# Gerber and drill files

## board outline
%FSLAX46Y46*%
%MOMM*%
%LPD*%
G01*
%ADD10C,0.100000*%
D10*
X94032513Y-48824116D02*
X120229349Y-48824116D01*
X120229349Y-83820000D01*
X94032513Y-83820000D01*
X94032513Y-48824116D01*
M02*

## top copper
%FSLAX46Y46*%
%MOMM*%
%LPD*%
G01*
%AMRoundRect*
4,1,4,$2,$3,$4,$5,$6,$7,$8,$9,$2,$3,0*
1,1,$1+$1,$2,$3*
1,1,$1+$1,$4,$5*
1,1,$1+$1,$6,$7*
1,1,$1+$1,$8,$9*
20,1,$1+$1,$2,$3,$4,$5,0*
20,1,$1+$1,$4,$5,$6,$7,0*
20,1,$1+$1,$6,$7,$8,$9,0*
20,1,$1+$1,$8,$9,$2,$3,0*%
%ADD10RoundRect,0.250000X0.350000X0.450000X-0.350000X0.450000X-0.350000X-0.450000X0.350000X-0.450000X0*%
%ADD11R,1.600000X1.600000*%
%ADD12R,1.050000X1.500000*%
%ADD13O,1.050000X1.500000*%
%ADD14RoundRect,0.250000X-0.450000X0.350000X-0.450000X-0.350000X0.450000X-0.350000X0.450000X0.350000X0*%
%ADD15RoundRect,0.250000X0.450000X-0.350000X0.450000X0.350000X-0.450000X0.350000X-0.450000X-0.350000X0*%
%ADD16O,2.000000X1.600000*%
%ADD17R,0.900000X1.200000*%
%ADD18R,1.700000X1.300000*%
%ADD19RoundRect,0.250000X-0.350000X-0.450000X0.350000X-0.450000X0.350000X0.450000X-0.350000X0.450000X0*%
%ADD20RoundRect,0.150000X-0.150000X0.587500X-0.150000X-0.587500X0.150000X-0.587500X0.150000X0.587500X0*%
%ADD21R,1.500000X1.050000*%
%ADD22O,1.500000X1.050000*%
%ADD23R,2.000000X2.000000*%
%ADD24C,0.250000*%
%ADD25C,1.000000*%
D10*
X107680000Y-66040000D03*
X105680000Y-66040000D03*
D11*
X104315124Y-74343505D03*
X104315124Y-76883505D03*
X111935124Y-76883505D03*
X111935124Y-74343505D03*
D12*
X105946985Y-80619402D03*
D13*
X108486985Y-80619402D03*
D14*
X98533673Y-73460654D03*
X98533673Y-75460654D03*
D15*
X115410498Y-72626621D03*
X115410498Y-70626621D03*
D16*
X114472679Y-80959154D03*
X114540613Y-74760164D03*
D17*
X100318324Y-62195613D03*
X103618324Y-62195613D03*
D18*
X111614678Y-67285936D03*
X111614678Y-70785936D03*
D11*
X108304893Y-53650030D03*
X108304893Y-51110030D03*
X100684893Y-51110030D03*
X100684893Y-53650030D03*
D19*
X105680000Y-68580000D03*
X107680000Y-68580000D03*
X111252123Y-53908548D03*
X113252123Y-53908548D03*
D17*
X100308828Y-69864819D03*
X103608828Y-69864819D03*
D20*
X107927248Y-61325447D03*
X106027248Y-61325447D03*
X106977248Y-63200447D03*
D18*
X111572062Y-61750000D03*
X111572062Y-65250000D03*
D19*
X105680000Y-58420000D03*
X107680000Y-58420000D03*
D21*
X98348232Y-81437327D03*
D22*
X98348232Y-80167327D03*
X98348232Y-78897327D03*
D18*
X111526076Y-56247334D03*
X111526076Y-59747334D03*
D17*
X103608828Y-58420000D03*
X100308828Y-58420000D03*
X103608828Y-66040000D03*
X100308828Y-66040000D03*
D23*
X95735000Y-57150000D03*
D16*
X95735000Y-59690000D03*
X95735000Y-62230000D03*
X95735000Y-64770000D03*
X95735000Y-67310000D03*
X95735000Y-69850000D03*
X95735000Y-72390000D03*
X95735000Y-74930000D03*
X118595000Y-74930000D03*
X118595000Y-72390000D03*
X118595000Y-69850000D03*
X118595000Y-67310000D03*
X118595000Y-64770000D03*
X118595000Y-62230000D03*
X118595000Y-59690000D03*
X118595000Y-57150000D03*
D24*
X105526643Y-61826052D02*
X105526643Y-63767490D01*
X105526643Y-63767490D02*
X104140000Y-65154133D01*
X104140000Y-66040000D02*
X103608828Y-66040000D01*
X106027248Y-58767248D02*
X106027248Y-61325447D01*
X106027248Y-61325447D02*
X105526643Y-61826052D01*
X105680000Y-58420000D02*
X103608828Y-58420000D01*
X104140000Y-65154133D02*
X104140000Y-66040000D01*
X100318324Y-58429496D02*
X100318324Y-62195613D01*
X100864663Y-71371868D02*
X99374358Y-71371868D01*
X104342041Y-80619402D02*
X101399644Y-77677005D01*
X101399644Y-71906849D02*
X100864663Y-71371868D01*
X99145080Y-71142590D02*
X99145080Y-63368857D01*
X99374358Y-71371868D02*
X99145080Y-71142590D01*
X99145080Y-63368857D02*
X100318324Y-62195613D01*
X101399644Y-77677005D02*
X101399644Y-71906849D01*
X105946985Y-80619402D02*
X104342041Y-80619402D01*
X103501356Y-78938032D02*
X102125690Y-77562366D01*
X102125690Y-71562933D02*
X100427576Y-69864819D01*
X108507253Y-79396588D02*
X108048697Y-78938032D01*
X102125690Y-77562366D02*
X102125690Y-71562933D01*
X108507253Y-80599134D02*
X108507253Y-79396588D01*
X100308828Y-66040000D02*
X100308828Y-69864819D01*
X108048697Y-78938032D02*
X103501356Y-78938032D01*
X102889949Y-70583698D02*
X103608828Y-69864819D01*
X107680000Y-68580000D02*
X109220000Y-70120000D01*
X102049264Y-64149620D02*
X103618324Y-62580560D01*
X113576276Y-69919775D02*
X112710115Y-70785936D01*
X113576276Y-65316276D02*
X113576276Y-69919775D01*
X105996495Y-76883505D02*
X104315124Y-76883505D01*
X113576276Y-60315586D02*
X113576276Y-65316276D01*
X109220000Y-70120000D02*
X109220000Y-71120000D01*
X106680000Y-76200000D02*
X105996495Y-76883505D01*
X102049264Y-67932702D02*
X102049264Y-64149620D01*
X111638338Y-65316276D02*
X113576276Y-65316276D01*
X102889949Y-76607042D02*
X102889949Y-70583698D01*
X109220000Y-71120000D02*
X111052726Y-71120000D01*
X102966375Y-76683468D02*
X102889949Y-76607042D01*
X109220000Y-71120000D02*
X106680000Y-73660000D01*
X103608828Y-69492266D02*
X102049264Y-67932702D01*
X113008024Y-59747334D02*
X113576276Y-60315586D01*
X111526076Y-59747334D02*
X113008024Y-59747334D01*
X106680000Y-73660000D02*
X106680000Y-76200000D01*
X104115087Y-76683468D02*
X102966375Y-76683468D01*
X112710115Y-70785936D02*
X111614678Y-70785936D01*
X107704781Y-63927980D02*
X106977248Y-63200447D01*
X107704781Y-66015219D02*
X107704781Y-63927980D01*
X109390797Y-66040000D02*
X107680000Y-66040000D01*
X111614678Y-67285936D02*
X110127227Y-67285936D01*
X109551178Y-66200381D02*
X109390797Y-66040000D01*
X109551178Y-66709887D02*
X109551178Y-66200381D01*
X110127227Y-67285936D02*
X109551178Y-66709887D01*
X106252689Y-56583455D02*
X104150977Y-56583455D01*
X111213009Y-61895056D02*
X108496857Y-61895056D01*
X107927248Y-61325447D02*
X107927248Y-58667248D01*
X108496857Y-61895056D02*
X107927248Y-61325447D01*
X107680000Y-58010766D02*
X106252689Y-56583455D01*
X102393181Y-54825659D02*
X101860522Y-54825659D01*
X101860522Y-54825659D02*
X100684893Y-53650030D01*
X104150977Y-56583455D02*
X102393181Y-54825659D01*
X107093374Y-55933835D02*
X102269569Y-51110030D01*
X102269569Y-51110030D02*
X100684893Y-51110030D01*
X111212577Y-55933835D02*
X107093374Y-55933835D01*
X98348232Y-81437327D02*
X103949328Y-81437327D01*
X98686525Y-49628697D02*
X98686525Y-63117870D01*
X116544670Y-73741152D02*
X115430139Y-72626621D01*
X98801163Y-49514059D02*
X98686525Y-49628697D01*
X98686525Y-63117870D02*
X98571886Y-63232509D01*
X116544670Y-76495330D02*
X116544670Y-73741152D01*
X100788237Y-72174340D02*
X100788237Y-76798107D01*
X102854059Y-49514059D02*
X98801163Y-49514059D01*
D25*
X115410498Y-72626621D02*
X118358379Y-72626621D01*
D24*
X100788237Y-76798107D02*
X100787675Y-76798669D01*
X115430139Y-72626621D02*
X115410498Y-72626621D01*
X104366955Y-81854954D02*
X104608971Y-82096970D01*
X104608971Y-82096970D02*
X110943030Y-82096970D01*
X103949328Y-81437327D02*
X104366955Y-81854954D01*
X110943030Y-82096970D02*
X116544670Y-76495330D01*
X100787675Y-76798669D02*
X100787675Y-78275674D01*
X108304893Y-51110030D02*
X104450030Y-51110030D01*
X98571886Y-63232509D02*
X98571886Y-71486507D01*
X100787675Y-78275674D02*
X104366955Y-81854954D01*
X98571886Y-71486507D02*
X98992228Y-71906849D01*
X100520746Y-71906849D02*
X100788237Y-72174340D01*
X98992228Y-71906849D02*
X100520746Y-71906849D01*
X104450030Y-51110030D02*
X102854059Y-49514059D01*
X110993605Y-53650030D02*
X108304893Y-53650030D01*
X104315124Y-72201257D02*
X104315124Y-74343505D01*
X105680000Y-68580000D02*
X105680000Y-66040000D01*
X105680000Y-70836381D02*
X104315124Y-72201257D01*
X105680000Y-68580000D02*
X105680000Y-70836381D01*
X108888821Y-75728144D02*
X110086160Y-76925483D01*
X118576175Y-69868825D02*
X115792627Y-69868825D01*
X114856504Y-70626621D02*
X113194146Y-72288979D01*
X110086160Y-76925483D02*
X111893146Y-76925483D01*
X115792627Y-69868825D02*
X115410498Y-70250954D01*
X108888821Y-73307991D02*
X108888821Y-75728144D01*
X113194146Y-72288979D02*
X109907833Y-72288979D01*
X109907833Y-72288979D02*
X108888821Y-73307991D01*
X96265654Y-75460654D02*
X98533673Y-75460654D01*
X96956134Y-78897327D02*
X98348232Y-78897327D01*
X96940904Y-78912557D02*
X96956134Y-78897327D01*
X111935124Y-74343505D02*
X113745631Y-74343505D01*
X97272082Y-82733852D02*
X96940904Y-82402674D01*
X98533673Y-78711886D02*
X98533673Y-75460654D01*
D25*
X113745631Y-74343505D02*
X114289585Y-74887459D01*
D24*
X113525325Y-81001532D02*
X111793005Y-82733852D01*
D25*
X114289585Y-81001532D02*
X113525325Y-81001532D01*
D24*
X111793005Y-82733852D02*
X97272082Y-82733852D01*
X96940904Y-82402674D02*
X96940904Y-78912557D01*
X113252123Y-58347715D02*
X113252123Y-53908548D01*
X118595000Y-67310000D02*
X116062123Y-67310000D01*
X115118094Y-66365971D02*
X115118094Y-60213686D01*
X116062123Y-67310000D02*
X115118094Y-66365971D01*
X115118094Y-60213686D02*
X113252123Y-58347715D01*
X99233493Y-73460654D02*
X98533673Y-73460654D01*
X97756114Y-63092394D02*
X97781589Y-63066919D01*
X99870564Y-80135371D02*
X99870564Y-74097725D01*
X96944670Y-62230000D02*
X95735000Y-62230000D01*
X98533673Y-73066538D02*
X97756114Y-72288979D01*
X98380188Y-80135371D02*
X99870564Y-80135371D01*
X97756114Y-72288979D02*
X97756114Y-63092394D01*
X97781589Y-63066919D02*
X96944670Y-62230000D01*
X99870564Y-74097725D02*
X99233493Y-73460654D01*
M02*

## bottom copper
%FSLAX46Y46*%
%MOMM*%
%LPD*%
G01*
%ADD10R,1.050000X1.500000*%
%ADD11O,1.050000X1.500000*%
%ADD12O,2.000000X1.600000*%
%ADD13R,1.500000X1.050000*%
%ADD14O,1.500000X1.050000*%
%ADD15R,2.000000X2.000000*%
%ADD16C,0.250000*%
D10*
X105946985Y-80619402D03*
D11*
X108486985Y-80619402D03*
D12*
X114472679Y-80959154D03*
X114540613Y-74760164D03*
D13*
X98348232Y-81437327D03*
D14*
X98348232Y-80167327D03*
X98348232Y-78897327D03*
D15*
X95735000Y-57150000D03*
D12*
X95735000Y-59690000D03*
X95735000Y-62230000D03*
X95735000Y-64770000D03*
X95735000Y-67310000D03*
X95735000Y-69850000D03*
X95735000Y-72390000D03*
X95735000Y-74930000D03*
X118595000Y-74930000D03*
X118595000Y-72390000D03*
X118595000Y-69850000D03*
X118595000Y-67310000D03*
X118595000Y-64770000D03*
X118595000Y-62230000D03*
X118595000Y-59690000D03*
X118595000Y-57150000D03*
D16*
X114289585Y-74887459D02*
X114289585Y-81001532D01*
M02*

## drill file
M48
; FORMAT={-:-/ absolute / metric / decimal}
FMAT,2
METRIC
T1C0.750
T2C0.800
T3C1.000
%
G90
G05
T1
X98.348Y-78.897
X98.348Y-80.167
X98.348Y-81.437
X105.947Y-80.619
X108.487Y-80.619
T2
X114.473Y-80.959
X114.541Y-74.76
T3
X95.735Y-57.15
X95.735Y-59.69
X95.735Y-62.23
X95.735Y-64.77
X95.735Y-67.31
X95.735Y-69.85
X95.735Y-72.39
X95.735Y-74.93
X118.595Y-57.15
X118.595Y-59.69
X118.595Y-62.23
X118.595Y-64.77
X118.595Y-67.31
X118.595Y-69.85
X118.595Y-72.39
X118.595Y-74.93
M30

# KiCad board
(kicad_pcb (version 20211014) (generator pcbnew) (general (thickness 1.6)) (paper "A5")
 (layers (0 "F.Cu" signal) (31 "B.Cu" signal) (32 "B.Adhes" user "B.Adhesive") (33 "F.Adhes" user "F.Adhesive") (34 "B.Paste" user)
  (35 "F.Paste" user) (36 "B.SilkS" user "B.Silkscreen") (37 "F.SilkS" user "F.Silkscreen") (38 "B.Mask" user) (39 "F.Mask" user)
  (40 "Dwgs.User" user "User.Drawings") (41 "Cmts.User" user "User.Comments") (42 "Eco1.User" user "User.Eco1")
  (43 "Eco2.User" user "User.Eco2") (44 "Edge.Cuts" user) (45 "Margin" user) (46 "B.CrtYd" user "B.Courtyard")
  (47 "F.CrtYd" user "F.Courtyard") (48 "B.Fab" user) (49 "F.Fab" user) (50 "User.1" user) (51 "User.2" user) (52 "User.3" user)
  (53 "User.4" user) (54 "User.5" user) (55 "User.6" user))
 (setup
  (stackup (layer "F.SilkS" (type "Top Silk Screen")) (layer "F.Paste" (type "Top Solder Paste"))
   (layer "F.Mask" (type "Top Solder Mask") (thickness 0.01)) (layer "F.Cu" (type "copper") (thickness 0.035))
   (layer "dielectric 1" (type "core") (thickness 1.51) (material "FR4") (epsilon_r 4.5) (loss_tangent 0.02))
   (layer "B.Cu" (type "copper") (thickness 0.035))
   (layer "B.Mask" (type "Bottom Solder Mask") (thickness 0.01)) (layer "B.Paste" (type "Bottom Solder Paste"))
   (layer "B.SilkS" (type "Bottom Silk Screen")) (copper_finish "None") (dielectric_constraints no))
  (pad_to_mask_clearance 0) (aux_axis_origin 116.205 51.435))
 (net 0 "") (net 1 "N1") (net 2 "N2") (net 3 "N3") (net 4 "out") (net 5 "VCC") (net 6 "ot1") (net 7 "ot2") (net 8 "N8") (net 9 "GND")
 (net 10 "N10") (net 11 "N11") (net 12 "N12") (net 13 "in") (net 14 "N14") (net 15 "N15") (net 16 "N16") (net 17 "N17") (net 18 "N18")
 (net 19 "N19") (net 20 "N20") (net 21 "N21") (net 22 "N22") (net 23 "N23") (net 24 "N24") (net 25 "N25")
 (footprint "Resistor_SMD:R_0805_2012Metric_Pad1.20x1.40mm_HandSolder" (layer "F.Cu") (at 106.68 66.04 180)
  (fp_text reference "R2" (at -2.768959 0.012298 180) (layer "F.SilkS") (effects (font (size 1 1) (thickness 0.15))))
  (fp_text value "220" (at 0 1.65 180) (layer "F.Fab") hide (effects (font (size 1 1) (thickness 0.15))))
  (pad "1" smd roundrect (at -1 0 180) (size 1.2 1.4) (layers "F.Cu" "F.Paste" "F.Mask") (roundrect_rratio 0.2083333333) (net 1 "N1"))
  (pad "2" smd roundrect (at 1 0 180) (size 1.2 1.4) (layers "F.Cu" "F.Paste" "F.Mask") (roundrect_rratio 0.2083333333) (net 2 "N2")))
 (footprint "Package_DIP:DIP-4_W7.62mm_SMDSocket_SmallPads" (layer "F.Cu") (at 108.125124 75.613505)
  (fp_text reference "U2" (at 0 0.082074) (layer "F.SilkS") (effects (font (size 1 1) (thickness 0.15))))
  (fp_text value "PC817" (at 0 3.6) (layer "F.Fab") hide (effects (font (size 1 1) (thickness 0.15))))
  (pad "1" smd rect (at -3.81 -1.27) (size 1.6 1.6) (layers "F.Cu" "F.Paste" "F.Mask") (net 2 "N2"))
  (pad "2" smd rect (at -3.81 1.27) (size 1.6 1.6) (layers "F.Cu" "F.Paste" "F.Mask") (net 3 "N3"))
  (pad "3" smd rect (at 3.81 1.27) (size 1.6 1.6) (layers "F.Cu" "F.Paste" "F.Mask") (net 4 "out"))
  (pad "4" smd rect (at 3.81 -1.27) (size 1.6 1.6) (layers "F.Cu" "F.Paste" "F.Mask") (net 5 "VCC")))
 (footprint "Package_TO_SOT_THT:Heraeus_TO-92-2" (layer "F.Cu") (at 105.946985 80.619402)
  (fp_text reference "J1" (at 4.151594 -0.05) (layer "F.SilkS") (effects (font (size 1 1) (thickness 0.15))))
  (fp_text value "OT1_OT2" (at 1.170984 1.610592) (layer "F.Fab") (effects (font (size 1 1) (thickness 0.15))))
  (pad "1" thru_hole rect (at 0 0) (size 1.05 1.5) (drill 0.75) (layers *.Cu *.Mask) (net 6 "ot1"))
  (pad "2" thru_hole oval (at 2.54 0) (size 1.05 1.5) (drill 0.75) (layers *.Cu *.Mask) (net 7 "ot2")))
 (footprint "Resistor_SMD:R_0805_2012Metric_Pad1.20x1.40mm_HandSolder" (layer "F.Cu") (at 98.533673 74.460654 -90)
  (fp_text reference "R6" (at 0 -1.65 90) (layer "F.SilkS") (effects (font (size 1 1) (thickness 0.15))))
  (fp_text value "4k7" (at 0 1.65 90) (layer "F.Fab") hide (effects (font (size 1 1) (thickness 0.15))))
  (pad "1" smd roundrect (at -1 0 270) (size 1.2 1.4) (layers "F.Cu" "F.Paste" "F.Mask") (roundrect_rratio 0.2083333333) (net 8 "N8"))
  (pad "2" smd roundrect (at 1 0 270) (size 1.2 1.4) (layers "F.Cu" "F.Paste" "F.Mask") (roundrect_rratio 0.2083333333) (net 5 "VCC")))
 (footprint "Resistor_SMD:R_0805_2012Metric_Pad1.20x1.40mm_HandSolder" (layer "F.Cu") (at 115.410498 71.626621 90)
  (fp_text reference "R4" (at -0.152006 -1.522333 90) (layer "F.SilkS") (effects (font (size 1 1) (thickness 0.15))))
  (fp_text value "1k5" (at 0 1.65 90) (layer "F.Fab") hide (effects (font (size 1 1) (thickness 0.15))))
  (pad "1" smd roundrect (at -1 0 90) (size 1.2 1.4) (layers "F.Cu" "F.Paste" "F.Mask") (roundrect_rratio 0.2083333333) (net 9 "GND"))
  (pad "2" smd roundrect (at 1 0 90) (size 1.2 1.4) (layers "F.Cu" "F.Paste" "F.Mask") (roundrect_rratio 0.2083333333) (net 4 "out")))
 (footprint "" (layer "F.Cu") (at 114.472679 80.959154)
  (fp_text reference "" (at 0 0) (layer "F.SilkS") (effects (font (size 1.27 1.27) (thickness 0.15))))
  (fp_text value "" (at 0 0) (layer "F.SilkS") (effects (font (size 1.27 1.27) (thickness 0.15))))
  (pad "001" thru_hole oval (at 0 0) (size 2 1.6) (drill 0.8) (layers *.Cu *.Mask) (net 5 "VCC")))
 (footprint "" (layer "F.Cu") (at 114.540613 74.760164)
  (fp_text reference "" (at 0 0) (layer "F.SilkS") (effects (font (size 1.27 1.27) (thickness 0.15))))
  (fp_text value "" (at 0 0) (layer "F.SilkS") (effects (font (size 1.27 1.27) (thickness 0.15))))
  (pad "001" thru_hole oval (at 0 0) (size 2 1.6) (drill 0.8) (layers *.Cu *.Mask) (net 5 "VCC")))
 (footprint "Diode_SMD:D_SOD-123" (layer "F.Cu") (at 101.968324 62.195613)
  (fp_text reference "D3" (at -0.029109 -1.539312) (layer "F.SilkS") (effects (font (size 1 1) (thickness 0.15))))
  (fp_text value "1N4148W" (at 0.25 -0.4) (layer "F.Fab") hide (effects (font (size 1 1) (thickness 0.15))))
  (pad "1" smd rect (at -1.65 0) (size 0.9 1.2) (layers "F.Cu" "F.Paste" "F.Mask") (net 3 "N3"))
  (pad "2" smd rect (at 1.65 0) (size 0.9 1.2) (layers "F.Cu" "F.Paste" "F.Mask") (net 6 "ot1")))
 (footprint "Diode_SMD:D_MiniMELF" (layer "F.Cu") (at 111.614678 69.035936 -90)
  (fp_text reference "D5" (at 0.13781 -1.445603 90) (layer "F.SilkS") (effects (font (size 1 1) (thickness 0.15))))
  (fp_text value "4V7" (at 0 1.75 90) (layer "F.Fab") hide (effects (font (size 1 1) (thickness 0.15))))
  (pad "1" smd rect (at -1.75 0 270) (size 1.3 1.7) (layers "F.Cu" "F.Paste" "F.Mask") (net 1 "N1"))
  (pad "2" smd rect (at 1.75 0 270) (size 1.3 1.7) (layers "F.Cu" "F.Paste" "F.Mask") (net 3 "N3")))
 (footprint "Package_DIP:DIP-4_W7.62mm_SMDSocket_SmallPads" (layer "F.Cu") (at 104.494893 52.38003 180)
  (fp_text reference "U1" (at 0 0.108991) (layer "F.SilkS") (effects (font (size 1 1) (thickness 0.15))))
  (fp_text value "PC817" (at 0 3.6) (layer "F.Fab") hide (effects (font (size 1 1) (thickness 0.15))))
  (pad "1" smd rect (at -3.81 -1.27 180) (size 1.6 1.6) (layers "F.Cu" "F.Paste" "F.Mask") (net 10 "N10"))
  (pad "2" smd rect (at -3.81 1.27 180) (size 1.6 1.6) (layers "F.Cu" "F.Paste" "F.Mask") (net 9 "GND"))
  (pad "3" smd rect (at 3.81 1.27 180) (size 1.6 1.6) (layers "F.Cu" "F.Paste" "F.Mask") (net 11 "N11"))
  (pad "4" smd rect (at 3.81 -1.27 180) (size 1.6 1.6) (layers "F.Cu" "F.Paste" "F.Mask") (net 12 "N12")))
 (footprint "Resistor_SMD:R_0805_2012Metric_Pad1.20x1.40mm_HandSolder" (layer "F.Cu") (at 106.68 68.58)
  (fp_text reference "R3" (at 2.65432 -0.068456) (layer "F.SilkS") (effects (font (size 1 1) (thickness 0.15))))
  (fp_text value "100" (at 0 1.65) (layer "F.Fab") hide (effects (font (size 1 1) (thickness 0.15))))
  (pad "1" smd roundrect (at -1 0) (size 1.2 1.4) (layers "F.Cu" "F.Paste" "F.Mask") (roundrect_rratio 0.2083333333) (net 2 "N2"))
  (pad "2" smd roundrect (at 1 0) (size 1.2 1.4) (layers "F.Cu" "F.Paste" "F.Mask") (roundrect_rratio 0.2083333333) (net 3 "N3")))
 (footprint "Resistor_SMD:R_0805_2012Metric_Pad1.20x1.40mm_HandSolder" (layer "F.Cu") (at 112.252123 53.908548)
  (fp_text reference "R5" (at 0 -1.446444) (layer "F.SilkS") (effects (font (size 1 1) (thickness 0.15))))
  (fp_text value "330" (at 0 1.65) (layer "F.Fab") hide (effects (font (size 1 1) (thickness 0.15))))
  (pad "1" smd roundrect (at -1 0) (size 1.2 1.4) (layers "F.Cu" "F.Paste" "F.Mask") (roundrect_rratio 0.2083333333) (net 10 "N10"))
  (pad "2" smd roundrect (at 1 0) (size 1.2 1.4) (layers "F.Cu" "F.Paste" "F.Mask") (roundrect_rratio 0.2083333333) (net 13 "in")))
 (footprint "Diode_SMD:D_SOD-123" (layer "F.Cu") (at 101.958828 69.864819)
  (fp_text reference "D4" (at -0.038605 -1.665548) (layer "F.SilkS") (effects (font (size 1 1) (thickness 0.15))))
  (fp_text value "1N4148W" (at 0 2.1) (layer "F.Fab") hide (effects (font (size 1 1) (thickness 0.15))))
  (pad "1" smd rect (at -1.65 0) (size 0.9 1.2) (layers "F.Cu" "F.Paste" "F.Mask") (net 3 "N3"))
  (pad "2" smd rect (at 1.65 0) (size 0.9 1.2) (layers "F.Cu" "F.Paste" "F.Mask") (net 7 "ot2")))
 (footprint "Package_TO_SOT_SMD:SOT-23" (layer "F.Cu") (at 106.977248 62.262947 -90)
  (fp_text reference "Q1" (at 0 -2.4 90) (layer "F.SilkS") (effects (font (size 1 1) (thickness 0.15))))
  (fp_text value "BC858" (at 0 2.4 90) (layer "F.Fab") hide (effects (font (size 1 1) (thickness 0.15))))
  (pad "1" smd roundrect (at -0.9375 -0.95 270) (size 1.475 0.6) (layers "F.Cu" "F.Paste" "F.Mask") (roundrect_rratio 0.25) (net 12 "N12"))
  (pad "2" smd roundrect (at -0.9375 0.95 270) (size 1.475 0.6) (layers "F.Cu" "F.Paste" "F.Mask") (roundrect_rratio 0.25) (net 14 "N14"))
  (pad "3" smd roundrect (at 0.9375 0 270) (size 1.475 0.6) (layers "F.Cu" "F.Paste" "F.Mask") (roundrect_rratio 0.25) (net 1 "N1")))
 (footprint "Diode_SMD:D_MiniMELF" (layer "F.Cu") (at 111.572062 63.5 -90)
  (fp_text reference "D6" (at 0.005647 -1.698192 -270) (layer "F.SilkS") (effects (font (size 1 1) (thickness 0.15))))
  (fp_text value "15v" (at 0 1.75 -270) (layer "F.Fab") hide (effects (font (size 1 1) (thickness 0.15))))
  (pad "1" smd rect (at -1.75 0 270) (size 1.3 1.7) (layers "F.Cu" "F.Paste" "F.Mask") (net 12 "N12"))
  (pad "2" smd rect (at 1.75 0 270) (size 1.3 1.7) (layers "F.Cu" "F.Paste" "F.Mask") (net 3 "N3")))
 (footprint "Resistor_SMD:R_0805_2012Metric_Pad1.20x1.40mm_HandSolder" (layer "F.Cu") (at 106.68 58.42)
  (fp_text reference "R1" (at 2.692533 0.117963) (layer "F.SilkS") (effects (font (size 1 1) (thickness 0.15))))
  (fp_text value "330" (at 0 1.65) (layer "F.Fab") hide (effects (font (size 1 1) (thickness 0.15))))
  (pad "1" smd roundrect (at -1 0) (size 1.2 1.4) (layers "F.Cu" "F.Paste" "F.Mask") (roundrect_rratio 0.2083333333) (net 14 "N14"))
  (pad "2" smd roundrect (at 1 0) (size 1.2 1.4) (layers "F.Cu" "F.Paste" "F.Mask") (roundrect_rratio 0.2083333333) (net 12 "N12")))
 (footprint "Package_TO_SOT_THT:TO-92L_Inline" (layer "F.Cu") (at 98.348232 81.437327 90)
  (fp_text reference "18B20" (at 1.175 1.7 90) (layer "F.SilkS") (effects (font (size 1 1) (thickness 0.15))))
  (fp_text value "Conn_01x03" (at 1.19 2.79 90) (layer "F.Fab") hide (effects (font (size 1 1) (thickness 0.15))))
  (pad "1" thru_hole rect (at 0 0 90) (size 1.05 1.5) (drill 0.75) (layers *.Cu *.Mask) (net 9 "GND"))
  (pad "2" thru_hole oval (at 1.27 0 90) (size 1.05 1.5) (drill 0.75) (layers *.Cu *.Mask) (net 8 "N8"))
  (pad "3" thru_hole oval (at 2.54 0 90) (size 1.05 1.5) (drill 0.75) (layers *.Cu *.Mask) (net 5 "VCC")))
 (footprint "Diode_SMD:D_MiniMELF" (layer "F.Cu") (at 111.526076 57.997334 -90)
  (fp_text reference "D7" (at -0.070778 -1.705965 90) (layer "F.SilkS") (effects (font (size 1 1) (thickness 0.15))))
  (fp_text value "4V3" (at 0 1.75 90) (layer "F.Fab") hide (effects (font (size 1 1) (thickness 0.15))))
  (pad "1" smd rect (at -1.75 0 270) (size 1.3 1.7) (layers "F.Cu" "F.Paste" "F.Mask") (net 11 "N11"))
  (pad "2" smd rect (at 1.75 0 270) (size 1.3 1.7) (layers "F.Cu" "F.Paste" "F.Mask") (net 3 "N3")))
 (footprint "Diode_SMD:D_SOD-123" (layer "F.Cu") (at 101.958828 58.42 180)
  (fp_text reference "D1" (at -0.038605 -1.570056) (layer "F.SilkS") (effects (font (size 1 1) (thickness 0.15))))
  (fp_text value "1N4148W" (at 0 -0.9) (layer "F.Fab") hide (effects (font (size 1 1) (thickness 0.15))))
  (pad "1" smd rect (at -1.65 0 180) (size 0.9 1.2) (layers "F.Cu" "F.Paste" "F.Mask") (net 14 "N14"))
  (pad "2" smd rect (at 1.65 0 180) (size 0.9 1.2) (layers "F.Cu" "F.Paste" "F.Mask") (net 6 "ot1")))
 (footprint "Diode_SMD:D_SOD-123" (layer "F.Cu") (at 101.958828 66.04 180)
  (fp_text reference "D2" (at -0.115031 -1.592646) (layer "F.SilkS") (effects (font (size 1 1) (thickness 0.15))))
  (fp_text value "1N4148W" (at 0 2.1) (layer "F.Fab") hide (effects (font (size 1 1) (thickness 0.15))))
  (pad "1" smd rect (at -1.65 0 180) (size 0.9 1.2) (layers "F.Cu" "F.Paste" "F.Mask") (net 14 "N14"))
  (pad "2" smd rect (at 1.65 0 180) (size 0.9 1.2) (layers "F.Cu" "F.Paste" "F.Mask") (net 7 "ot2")))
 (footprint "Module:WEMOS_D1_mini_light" (layer "F.Cu") (at 95.735 57.15)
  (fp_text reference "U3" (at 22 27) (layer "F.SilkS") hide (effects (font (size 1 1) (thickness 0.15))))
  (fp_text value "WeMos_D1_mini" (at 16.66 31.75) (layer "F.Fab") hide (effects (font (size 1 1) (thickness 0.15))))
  (pad "1" thru_hole rect (at 0 0) (size 2 2) (drill 1) (layers *.Cu *.Mask) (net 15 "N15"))
  (pad "2" thru_hole oval (at 0 2.54) (size 2 1.6) (drill 1) (layers *.Cu *.Mask) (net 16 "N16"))
  (pad "3" thru_hole oval (at 0 5.08) (size 2 1.6) (drill 1) (layers *.Cu *.Mask) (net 8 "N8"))
  (pad "4" thru_hole oval (at 0 7.62) (size 2 1.6) (drill 1) (layers *.Cu *.Mask) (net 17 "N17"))
  (pad "5" thru_hole oval (at 0 10.16) (size 2 1.6) (drill 1) (layers *.Cu *.Mask) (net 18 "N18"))
  (pad "6" thru_hole oval (at 0 12.7) (size 2 1.6) (drill 1) (layers *.Cu *.Mask) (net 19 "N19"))
  (pad "7" thru_hole oval (at 0 15.24) (size 2 1.6) (drill 1) (layers *.Cu *.Mask) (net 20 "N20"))
  (pad "8" thru_hole oval (at 0 17.78) (size 2 1.6) (drill 1) (layers *.Cu *.Mask) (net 5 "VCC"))
  (pad "9" thru_hole oval (at 22.86 17.78) (size 2 1.6) (drill 1) (layers *.Cu *.Mask) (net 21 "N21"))
  (pad "10" thru_hole oval (at 22.86 15.24) (size 2 1.6) (drill 1) (layers *.Cu *.Mask) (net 9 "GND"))
  (pad "11" thru_hole oval (at 22.86 12.7) (size 2 1.6) (drill 1) (layers *.Cu *.Mask) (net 4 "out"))
  (pad "12" thru_hole oval (at 22.86 10.16) (size 2 1.6) (drill 1) (layers *.Cu *.Mask) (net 13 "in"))
  (pad "13" thru_hole oval (at 22.86 7.62) (size 2 1.6) (drill 1) (layers *.Cu *.Mask) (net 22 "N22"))
  (pad "14" thru_hole oval (at 22.86 5.08) (size 2 1.6) (drill 1) (layers *.Cu *.Mask) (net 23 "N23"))
  (pad "15" thru_hole oval (at 22.86 2.54) (size 2 1.6) (drill 1) (layers *.Cu *.Mask) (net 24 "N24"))
  (pad "16" thru_hole oval (at 22.86 0) (size 2 1.6) (drill 1) (layers *.Cu *.Mask) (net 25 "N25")))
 (gr_rect (start 120.229349 83.82) (end 94.032513 48.824116) (layer "Edge.Cuts") (width 0.1) (fill none))
 (segment (start 105.526643 61.826052) (end 105.526643 63.76749) (width 0.25) (layer "F.Cu") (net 14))
 (segment (start 105.526643 63.76749) (end 104.14 65.154133) (width 0.25) (layer "F.Cu") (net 14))
 (segment (start 104.14 66.04) (end 103.608828 66.04) (width 0.25) (layer "F.Cu") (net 14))
 (segment (start 106.027248 58.767248) (end 106.027248 61.325447) (width 0.25) (layer "F.Cu") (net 14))
 (segment (start 106.027248 61.325447) (end 105.526643 61.826052) (width 0.25) (layer "F.Cu") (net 14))
 (segment (start 105.68 58.42) (end 103.608828 58.42) (width 0.25) (layer "F.Cu") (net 14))
 (segment (start 104.14 65.154133) (end 104.14 66.04) (width 0.25) (layer "F.Cu") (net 14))
 (segment (start 100.318324 58.429496) (end 100.318324 62.195613) (width 0.25) (layer "F.Cu") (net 6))
 (segment (start 100.864663 71.371868) (end 99.374358 71.371868) (width 0.25) (layer "F.Cu") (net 6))
 (segment (start 104.342041 80.619402) (end 101.399644 77.677005) (width 0.25) (layer "F.Cu") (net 6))
 (segment (start 101.399644 71.906849) (end 100.864663 71.371868) (width 0.25) (layer "F.Cu") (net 6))
 (segment (start 99.14508 71.14259) (end 99.14508 63.368857) (width 0.25) (layer "F.Cu") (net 6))
 (segment (start 99.374358 71.371868) (end 99.14508 71.14259) (width 0.25) (layer "F.Cu") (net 6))
 (segment (start 99.14508 63.368857) (end 100.318324 62.195613) (width 0.25) (layer "F.Cu") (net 6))
 (segment (start 101.399644 77.677005) (end 101.399644 71.906849) (width 0.25) (layer "F.Cu") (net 6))
 (segment (start 105.946985 80.619402) (end 104.342041 80.619402) (width 0.25) (layer "F.Cu") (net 6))
 (segment (start 103.501356 78.938032) (end 102.12569 77.562366) (width 0.25) (layer "F.Cu") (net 7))
 (segment (start 102.12569 71.562933) (end 100.427576 69.864819) (width 0.25) (layer "F.Cu") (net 7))
 (segment (start 108.507253 79.396588) (end 108.048697 78.938032) (width 0.25) (layer "F.Cu") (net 7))
 (segment (start 102.12569 77.562366) (end 102.12569 71.562933) (width 0.25) (layer "F.Cu") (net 7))
 (segment (start 108.507253 80.599134) (end 108.507253 79.396588) (width 0.25) (layer "F.Cu") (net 7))
 (segment (start 100.308828 66.04) (end 100.308828 69.864819) (width 0.25) (layer "F.Cu") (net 7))
 (segment (start 108.048697 78.938032) (end 103.501356 78.938032) (width 0.25) (layer "F.Cu") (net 7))
 (segment (start 102.889949 70.583698) (end 103.608828 69.864819) (width 0.25) (layer "F.Cu") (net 3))
 (segment (start 107.68 68.58) (end 109.22 70.12) (width 0.25) (layer "F.Cu") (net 3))
 (segment (start 102.049264 64.14962) (end 103.618324 62.58056) (width 0.25) (layer "F.Cu") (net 3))
 (segment (start 113.576276 69.919775) (end 112.710115 70.785936) (width 0.25) (layer "F.Cu") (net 3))
 (segment (start 113.576276 65.316276) (end 113.576276 69.919775) (width 0.25) (layer "F.Cu") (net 3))
 (segment (start 105.996495 76.883505) (end 104.315124 76.883505) (width 0.25) (layer "F.Cu") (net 3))
 (segment (start 113.576276 60.315586) (end 113.576276 65.316276) (width 0.25) (layer "F.Cu") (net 3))
 (segment (start 109.22 70.12) (end 109.22 71.12) (width 0.25) (layer "F.Cu") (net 3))
 (segment (start 106.68 76.2) (end 105.996495 76.883505) (width 0.25) (layer "F.Cu") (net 3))
 (segment (start 102.049264 67.932702) (end 102.049264 64.14962) (width 0.25) (layer "F.Cu") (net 3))
 (segment (start 111.638338 65.316276) (end 113.576276 65.316276) (width 0.25) (layer "F.Cu") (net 3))
 (segment (start 102.889949 76.607042) (end 102.889949 70.583698) (width 0.25) (layer "F.Cu") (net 3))
 (segment (start 109.22 71.12) (end 111.052726 71.12) (width 0.25) (layer "F.Cu") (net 3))
 (segment (start 102.966375 76.683468) (end 102.889949 76.607042) (width 0.25) (layer "F.Cu") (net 3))
 (segment (start 109.22 71.12) (end 106.68 73.66) (width 0.25) (layer "F.Cu") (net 3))
 (segment (start 103.608828 69.492266) (end 102.049264 67.932702) (width 0.25) (layer "F.Cu") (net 3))
 (segment (start 113.008024 59.747334) (end 113.576276 60.315586) (width 0.25) (layer "F.Cu") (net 3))
 (segment (start 111.526076 59.747334) (end 113.008024 59.747334) (width 0.25) (layer "F.Cu") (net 3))
 (segment (start 106.68 73.66) (end 106.68 76.2) (width 0.25) (layer "F.Cu") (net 3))
 (segment (start 104.115087 76.683468) (end 102.966375 76.683468) (width 0.25) (layer "F.Cu") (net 3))
 (segment (start 112.710115 70.785936) (end 111.614678 70.785936) (width 0.25) (layer "F.Cu") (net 3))
 (segment (start 107.704781 63.92798) (end 106.977248 63.200447) (width 0.25) (layer "F.Cu") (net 1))
 (segment (start 107.704781 66.015219) (end 107.704781 63.92798) (width 0.25) (layer "F.Cu") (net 1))
 (segment (start 109.390797 66.04) (end 107.68 66.04) (width 0.25) (layer "F.Cu") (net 1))
 (segment (start 111.614678 67.285936) (end 110.127227 67.285936) (width 0.25) (layer "F.Cu") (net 1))
 (segment (start 109.551178 66.200381) (end 109.390797 66.04) (width 0.25) (layer "F.Cu") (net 1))
 (segment (start 109.551178 66.709887) (end 109.551178 66.200381) (width 0.25) (layer "F.Cu") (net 1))
 (segment (start 110.127227 67.285936) (end 109.551178 66.709887) (width 0.25) (layer "F.Cu") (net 1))
 (segment (start 106.252689 56.583455) (end 104.150977 56.583455) (width 0.25) (layer "F.Cu") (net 12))
 (segment (start 111.213009 61.895056) (end 108.496857 61.895056) (width 0.25) (layer "F.Cu") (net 12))
 (segment (start 107.927248 61.325447) (end 107.927248 58.667248) (width 0.25) (layer "F.Cu") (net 12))
 (segment (start 108.496857 61.895056) (end 107.927248 61.325447) (width 0.25) (layer "F.Cu") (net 12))
 (segment (start 107.68 58.010766) (end 106.252689 56.583455) (width 0.25) (layer "F.Cu") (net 12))
 (segment (start 102.393181 54.825659) (end 101.860522 54.825659) (width 0.25) (layer "F.Cu") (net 12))
 (segment (start 101.860522 54.825659) (end 100.684893 53.65003) (width 0.25) (layer "F.Cu") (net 12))
 (segment (start 104.150977 56.583455) (end 102.393181 54.825659) (width 0.25) (layer "F.Cu") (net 12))
 (segment (start 107.093374 55.933835) (end 102.269569 51.11003) (width 0.25) (layer "F.Cu") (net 11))
 (segment (start 102.269569 51.11003) (end 100.684893 51.11003) (width 0.25) (layer "F.Cu") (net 11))
 (segment (start 111.212577 55.933835) (end 107.093374 55.933835) (width 0.25) (layer "F.Cu") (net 11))
 (segment (start 98.348232 81.437327) (end 103.949328 81.437327) (width 0.25) (layer "F.Cu") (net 9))
 (segment (start 98.686525 49.628697) (end 98.686525 63.11787) (width 0.25) (layer "F.Cu") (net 9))
 (segment (start 116.54467 73.741152) (end 115.430139 72.626621) (width 0.25) (layer "F.Cu") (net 9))
 (segment (start 98.801163 49.514059) (end 98.686525 49.628697) (width 0.25) (layer "F.Cu") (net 9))
 (segment (start 98.686525 63.11787) (end 98.571886 63.232509) (width 0.25) (layer "F.Cu") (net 9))
 (segment (start 116.54467 76.49533) (end 116.54467 73.741152) (width 0.25) (layer "F.Cu") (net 9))
 (segment (start 100.788237 72.17434) (end 100.788237 76.798107) (width 0.25) (layer "F.Cu") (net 9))
 (segment (start 102.854059 49.514059) (end 98.801163 49.514059) (width 0.25) (layer "F.Cu") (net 9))
 (segment (start 115.410498 72.626621) (end 118.358379 72.626621) (width 1) (layer "F.Cu") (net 9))
 (segment (start 100.788237 76.798107) (end 100.787675 76.798669) (width 0.25) (layer "F.Cu") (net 9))
 (segment (start 115.430139 72.626621) (end 115.410498 72.626621) (width 0.25) (layer "F.Cu") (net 9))
 (segment (start 104.366955 81.854954) (end 104.608971 82.09697) (width 0.25) (layer "F.Cu") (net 9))
 (segment (start 104.608971 82.09697) (end 110.94303 82.09697) (width 0.25) (layer "F.Cu") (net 9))
 (segment (start 103.949328 81.437327) (end 104.366955 81.854954) (width 0.25) (layer "F.Cu") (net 9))
 (segment (start 110.94303 82.09697) (end 116.54467 76.49533) (width 0.25) (layer "F.Cu") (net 9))
 (segment (start 100.787675 76.798669) (end 100.787675 78.275674) (width 0.25) (layer "F.Cu") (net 9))
 (segment (start 108.304893 51.11003) (end 104.45003 51.11003) (width 0.25) (layer "F.Cu") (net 9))
 (segment (start 98.571886 63.232509) (end 98.571886 71.486507) (width 0.25) (layer "F.Cu") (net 9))
 (segment (start 100.787675 78.275674) (end 104.366955 81.854954) (width 0.25) (layer "F.Cu") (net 9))
 (segment (start 98.571886 71.486507) (end 98.992228 71.906849) (width 0.25) (layer "F.Cu") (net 9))
 (segment (start 100.520746 71.906849) (end 100.788237 72.17434) (width 0.25) (layer "F.Cu") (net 9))
 (segment (start 98.992228 71.906849) (end 100.520746 71.906849) (width 0.25) (layer "F.Cu") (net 9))
 (segment (start 104.45003 51.11003) (end 102.854059 49.514059) (width 0.25) (layer "F.Cu") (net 9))
 (segment (start 110.993605 53.65003) (end 108.304893 53.65003) (width 0.25) (layer "F.Cu") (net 10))
 (segment (start 104.315124 72.201257) (end 104.315124 74.343505) (width 0.25) (layer "F.Cu") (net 2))
 (segment (start 105.68 68.58) (end 105.68 66.04) (width 0.25) (layer "F.Cu") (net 2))
 (segment (start 105.68 70.836381) (end 104.315124 72.201257) (width 0.25) (layer "F.Cu") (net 2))
 (segment (start 105.68 68.58) (end 105.68 70.836381) (width 0.25) (layer "F.Cu") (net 2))
 (segment (start 108.888821 75.728144) (end 110.08616 76.925483) (width 0.25) (layer "F.Cu") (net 4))
 (segment (start 118.576175 69.868825) (end 115.792627 69.868825) (width 0.25) (layer "F.Cu") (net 4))
 (segment (start 114.856504 70.626621) (end 113.194146 72.288979) (width 0.25) (layer "F.Cu") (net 4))
 (segment (start 110.08616 76.925483) (end 111.893146 76.925483) (width 0.25) (layer "F.Cu") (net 4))
 (segment (start 115.792627 69.868825) (end 115.410498 70.250954) (width 0.25) (layer "F.Cu") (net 4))
 (segment (start 108.888821 73.307991) (end 108.888821 75.728144) (width 0.25) (layer "F.Cu") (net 4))
 (segment (start 113.194146 72.288979) (end 109.907833 72.288979) (width 0.25) (layer "F.Cu") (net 4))
 (segment (start 109.907833 72.288979) (end 108.888821 73.307991) (width 0.25) (layer "F.Cu") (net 4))
 (segment (start 96.265654 75.460654) (end 98.533673 75.460654) (width 0.25) (layer "F.Cu") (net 5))
 (segment (start 96.956134 78.897327) (end 98.348232 78.897327) (width 0.25) (layer "F.Cu") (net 5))
 (segment (start 96.940904 78.912557) (end 96.956134 78.897327) (width 0.25) (layer "F.Cu") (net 5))
 (segment (start 111.935124 74.343505) (end 113.745631 74.343505) (width 0.25) (layer "F.Cu") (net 5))
 (segment (start 97.272082 82.733852) (end 96.940904 82.402674) (width 0.25) (layer "F.Cu") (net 5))
 (segment (start 98.533673 78.711886) (end 98.533673 75.460654) (width 0.25) (layer "F.Cu") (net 5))
 (segment (start 113.745631 74.343505) (end 114.289585 74.887459) (width 1) (layer "F.Cu") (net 5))
 (segment (start 113.525325 81.001532) (end 111.793005 82.733852) (width 0.25) (layer "F.Cu") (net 5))
 (segment (start 114.289585 81.001532) (end 113.525325 81.001532) (width 1) (layer "F.Cu") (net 5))
 (segment (start 111.793005 82.733852) (end 97.272082 82.733852) (width 0.25) (layer "F.Cu") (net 5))
 (segment (start 96.940904 82.402674) (end 96.940904 78.912557) (width 0.25) (layer "F.Cu") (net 5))
 (segment (start 114.289585 74.887459) (end 114.289585 81.001532) (width 0.25) (layer "B.Cu") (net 5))
 (segment (start 113.252123 58.347715) (end 113.252123 53.908548) (width 0.25) (layer "F.Cu") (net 13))
 (segment (start 118.595 67.31) (end 116.062123 67.31) (width 0.25) (layer "F.Cu") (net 13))
 (segment (start 115.118094 66.365971) (end 115.118094 60.213686) (width 0.25) (layer "F.Cu") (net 13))
 (segment (start 116.062123 67.31) (end 115.118094 66.365971) (width 0.25) (layer "F.Cu") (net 13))
 (segment (start 115.118094 60.213686) (end 113.252123 58.347715) (width 0.25) (layer "F.Cu") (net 13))
 (segment (start 99.233493 73.460654) (end 98.533673 73.460654) (width 0.25) (layer "F.Cu") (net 8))
 (segment (start 97.756114 63.092394) (end 97.781589 63.066919) (width 0.25) (layer "F.Cu") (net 8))
 (segment (start 99.870564 80.135371) (end 99.870564 74.097725) (width 0.25) (layer "F.Cu") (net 8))
 (segment (start 96.94467 62.23) (end 95.735 62.23) (width 0.25) (layer "F.Cu") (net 8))
 (segment (start 98.533673 73.066538) (end 97.756114 72.288979) (width 0.25) (layer "F.Cu") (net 8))
 (segment (start 98.380188 80.135371) (end 99.870564 80.135371) (width 0.25) (layer "F.Cu") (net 8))
 (segment (start 97.756114 72.288979) (end 97.756114 63.092394) (width 0.25) (layer "F.Cu") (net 8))
 (segment (start 97.781589 63.066919) (end 96.94467 62.23) (width 0.25) (layer "F.Cu") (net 8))
 (segment (start 99.870564 74.097725) (end 99.233493 73.460654) (width 0.25) (layer "F.Cu") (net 8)))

